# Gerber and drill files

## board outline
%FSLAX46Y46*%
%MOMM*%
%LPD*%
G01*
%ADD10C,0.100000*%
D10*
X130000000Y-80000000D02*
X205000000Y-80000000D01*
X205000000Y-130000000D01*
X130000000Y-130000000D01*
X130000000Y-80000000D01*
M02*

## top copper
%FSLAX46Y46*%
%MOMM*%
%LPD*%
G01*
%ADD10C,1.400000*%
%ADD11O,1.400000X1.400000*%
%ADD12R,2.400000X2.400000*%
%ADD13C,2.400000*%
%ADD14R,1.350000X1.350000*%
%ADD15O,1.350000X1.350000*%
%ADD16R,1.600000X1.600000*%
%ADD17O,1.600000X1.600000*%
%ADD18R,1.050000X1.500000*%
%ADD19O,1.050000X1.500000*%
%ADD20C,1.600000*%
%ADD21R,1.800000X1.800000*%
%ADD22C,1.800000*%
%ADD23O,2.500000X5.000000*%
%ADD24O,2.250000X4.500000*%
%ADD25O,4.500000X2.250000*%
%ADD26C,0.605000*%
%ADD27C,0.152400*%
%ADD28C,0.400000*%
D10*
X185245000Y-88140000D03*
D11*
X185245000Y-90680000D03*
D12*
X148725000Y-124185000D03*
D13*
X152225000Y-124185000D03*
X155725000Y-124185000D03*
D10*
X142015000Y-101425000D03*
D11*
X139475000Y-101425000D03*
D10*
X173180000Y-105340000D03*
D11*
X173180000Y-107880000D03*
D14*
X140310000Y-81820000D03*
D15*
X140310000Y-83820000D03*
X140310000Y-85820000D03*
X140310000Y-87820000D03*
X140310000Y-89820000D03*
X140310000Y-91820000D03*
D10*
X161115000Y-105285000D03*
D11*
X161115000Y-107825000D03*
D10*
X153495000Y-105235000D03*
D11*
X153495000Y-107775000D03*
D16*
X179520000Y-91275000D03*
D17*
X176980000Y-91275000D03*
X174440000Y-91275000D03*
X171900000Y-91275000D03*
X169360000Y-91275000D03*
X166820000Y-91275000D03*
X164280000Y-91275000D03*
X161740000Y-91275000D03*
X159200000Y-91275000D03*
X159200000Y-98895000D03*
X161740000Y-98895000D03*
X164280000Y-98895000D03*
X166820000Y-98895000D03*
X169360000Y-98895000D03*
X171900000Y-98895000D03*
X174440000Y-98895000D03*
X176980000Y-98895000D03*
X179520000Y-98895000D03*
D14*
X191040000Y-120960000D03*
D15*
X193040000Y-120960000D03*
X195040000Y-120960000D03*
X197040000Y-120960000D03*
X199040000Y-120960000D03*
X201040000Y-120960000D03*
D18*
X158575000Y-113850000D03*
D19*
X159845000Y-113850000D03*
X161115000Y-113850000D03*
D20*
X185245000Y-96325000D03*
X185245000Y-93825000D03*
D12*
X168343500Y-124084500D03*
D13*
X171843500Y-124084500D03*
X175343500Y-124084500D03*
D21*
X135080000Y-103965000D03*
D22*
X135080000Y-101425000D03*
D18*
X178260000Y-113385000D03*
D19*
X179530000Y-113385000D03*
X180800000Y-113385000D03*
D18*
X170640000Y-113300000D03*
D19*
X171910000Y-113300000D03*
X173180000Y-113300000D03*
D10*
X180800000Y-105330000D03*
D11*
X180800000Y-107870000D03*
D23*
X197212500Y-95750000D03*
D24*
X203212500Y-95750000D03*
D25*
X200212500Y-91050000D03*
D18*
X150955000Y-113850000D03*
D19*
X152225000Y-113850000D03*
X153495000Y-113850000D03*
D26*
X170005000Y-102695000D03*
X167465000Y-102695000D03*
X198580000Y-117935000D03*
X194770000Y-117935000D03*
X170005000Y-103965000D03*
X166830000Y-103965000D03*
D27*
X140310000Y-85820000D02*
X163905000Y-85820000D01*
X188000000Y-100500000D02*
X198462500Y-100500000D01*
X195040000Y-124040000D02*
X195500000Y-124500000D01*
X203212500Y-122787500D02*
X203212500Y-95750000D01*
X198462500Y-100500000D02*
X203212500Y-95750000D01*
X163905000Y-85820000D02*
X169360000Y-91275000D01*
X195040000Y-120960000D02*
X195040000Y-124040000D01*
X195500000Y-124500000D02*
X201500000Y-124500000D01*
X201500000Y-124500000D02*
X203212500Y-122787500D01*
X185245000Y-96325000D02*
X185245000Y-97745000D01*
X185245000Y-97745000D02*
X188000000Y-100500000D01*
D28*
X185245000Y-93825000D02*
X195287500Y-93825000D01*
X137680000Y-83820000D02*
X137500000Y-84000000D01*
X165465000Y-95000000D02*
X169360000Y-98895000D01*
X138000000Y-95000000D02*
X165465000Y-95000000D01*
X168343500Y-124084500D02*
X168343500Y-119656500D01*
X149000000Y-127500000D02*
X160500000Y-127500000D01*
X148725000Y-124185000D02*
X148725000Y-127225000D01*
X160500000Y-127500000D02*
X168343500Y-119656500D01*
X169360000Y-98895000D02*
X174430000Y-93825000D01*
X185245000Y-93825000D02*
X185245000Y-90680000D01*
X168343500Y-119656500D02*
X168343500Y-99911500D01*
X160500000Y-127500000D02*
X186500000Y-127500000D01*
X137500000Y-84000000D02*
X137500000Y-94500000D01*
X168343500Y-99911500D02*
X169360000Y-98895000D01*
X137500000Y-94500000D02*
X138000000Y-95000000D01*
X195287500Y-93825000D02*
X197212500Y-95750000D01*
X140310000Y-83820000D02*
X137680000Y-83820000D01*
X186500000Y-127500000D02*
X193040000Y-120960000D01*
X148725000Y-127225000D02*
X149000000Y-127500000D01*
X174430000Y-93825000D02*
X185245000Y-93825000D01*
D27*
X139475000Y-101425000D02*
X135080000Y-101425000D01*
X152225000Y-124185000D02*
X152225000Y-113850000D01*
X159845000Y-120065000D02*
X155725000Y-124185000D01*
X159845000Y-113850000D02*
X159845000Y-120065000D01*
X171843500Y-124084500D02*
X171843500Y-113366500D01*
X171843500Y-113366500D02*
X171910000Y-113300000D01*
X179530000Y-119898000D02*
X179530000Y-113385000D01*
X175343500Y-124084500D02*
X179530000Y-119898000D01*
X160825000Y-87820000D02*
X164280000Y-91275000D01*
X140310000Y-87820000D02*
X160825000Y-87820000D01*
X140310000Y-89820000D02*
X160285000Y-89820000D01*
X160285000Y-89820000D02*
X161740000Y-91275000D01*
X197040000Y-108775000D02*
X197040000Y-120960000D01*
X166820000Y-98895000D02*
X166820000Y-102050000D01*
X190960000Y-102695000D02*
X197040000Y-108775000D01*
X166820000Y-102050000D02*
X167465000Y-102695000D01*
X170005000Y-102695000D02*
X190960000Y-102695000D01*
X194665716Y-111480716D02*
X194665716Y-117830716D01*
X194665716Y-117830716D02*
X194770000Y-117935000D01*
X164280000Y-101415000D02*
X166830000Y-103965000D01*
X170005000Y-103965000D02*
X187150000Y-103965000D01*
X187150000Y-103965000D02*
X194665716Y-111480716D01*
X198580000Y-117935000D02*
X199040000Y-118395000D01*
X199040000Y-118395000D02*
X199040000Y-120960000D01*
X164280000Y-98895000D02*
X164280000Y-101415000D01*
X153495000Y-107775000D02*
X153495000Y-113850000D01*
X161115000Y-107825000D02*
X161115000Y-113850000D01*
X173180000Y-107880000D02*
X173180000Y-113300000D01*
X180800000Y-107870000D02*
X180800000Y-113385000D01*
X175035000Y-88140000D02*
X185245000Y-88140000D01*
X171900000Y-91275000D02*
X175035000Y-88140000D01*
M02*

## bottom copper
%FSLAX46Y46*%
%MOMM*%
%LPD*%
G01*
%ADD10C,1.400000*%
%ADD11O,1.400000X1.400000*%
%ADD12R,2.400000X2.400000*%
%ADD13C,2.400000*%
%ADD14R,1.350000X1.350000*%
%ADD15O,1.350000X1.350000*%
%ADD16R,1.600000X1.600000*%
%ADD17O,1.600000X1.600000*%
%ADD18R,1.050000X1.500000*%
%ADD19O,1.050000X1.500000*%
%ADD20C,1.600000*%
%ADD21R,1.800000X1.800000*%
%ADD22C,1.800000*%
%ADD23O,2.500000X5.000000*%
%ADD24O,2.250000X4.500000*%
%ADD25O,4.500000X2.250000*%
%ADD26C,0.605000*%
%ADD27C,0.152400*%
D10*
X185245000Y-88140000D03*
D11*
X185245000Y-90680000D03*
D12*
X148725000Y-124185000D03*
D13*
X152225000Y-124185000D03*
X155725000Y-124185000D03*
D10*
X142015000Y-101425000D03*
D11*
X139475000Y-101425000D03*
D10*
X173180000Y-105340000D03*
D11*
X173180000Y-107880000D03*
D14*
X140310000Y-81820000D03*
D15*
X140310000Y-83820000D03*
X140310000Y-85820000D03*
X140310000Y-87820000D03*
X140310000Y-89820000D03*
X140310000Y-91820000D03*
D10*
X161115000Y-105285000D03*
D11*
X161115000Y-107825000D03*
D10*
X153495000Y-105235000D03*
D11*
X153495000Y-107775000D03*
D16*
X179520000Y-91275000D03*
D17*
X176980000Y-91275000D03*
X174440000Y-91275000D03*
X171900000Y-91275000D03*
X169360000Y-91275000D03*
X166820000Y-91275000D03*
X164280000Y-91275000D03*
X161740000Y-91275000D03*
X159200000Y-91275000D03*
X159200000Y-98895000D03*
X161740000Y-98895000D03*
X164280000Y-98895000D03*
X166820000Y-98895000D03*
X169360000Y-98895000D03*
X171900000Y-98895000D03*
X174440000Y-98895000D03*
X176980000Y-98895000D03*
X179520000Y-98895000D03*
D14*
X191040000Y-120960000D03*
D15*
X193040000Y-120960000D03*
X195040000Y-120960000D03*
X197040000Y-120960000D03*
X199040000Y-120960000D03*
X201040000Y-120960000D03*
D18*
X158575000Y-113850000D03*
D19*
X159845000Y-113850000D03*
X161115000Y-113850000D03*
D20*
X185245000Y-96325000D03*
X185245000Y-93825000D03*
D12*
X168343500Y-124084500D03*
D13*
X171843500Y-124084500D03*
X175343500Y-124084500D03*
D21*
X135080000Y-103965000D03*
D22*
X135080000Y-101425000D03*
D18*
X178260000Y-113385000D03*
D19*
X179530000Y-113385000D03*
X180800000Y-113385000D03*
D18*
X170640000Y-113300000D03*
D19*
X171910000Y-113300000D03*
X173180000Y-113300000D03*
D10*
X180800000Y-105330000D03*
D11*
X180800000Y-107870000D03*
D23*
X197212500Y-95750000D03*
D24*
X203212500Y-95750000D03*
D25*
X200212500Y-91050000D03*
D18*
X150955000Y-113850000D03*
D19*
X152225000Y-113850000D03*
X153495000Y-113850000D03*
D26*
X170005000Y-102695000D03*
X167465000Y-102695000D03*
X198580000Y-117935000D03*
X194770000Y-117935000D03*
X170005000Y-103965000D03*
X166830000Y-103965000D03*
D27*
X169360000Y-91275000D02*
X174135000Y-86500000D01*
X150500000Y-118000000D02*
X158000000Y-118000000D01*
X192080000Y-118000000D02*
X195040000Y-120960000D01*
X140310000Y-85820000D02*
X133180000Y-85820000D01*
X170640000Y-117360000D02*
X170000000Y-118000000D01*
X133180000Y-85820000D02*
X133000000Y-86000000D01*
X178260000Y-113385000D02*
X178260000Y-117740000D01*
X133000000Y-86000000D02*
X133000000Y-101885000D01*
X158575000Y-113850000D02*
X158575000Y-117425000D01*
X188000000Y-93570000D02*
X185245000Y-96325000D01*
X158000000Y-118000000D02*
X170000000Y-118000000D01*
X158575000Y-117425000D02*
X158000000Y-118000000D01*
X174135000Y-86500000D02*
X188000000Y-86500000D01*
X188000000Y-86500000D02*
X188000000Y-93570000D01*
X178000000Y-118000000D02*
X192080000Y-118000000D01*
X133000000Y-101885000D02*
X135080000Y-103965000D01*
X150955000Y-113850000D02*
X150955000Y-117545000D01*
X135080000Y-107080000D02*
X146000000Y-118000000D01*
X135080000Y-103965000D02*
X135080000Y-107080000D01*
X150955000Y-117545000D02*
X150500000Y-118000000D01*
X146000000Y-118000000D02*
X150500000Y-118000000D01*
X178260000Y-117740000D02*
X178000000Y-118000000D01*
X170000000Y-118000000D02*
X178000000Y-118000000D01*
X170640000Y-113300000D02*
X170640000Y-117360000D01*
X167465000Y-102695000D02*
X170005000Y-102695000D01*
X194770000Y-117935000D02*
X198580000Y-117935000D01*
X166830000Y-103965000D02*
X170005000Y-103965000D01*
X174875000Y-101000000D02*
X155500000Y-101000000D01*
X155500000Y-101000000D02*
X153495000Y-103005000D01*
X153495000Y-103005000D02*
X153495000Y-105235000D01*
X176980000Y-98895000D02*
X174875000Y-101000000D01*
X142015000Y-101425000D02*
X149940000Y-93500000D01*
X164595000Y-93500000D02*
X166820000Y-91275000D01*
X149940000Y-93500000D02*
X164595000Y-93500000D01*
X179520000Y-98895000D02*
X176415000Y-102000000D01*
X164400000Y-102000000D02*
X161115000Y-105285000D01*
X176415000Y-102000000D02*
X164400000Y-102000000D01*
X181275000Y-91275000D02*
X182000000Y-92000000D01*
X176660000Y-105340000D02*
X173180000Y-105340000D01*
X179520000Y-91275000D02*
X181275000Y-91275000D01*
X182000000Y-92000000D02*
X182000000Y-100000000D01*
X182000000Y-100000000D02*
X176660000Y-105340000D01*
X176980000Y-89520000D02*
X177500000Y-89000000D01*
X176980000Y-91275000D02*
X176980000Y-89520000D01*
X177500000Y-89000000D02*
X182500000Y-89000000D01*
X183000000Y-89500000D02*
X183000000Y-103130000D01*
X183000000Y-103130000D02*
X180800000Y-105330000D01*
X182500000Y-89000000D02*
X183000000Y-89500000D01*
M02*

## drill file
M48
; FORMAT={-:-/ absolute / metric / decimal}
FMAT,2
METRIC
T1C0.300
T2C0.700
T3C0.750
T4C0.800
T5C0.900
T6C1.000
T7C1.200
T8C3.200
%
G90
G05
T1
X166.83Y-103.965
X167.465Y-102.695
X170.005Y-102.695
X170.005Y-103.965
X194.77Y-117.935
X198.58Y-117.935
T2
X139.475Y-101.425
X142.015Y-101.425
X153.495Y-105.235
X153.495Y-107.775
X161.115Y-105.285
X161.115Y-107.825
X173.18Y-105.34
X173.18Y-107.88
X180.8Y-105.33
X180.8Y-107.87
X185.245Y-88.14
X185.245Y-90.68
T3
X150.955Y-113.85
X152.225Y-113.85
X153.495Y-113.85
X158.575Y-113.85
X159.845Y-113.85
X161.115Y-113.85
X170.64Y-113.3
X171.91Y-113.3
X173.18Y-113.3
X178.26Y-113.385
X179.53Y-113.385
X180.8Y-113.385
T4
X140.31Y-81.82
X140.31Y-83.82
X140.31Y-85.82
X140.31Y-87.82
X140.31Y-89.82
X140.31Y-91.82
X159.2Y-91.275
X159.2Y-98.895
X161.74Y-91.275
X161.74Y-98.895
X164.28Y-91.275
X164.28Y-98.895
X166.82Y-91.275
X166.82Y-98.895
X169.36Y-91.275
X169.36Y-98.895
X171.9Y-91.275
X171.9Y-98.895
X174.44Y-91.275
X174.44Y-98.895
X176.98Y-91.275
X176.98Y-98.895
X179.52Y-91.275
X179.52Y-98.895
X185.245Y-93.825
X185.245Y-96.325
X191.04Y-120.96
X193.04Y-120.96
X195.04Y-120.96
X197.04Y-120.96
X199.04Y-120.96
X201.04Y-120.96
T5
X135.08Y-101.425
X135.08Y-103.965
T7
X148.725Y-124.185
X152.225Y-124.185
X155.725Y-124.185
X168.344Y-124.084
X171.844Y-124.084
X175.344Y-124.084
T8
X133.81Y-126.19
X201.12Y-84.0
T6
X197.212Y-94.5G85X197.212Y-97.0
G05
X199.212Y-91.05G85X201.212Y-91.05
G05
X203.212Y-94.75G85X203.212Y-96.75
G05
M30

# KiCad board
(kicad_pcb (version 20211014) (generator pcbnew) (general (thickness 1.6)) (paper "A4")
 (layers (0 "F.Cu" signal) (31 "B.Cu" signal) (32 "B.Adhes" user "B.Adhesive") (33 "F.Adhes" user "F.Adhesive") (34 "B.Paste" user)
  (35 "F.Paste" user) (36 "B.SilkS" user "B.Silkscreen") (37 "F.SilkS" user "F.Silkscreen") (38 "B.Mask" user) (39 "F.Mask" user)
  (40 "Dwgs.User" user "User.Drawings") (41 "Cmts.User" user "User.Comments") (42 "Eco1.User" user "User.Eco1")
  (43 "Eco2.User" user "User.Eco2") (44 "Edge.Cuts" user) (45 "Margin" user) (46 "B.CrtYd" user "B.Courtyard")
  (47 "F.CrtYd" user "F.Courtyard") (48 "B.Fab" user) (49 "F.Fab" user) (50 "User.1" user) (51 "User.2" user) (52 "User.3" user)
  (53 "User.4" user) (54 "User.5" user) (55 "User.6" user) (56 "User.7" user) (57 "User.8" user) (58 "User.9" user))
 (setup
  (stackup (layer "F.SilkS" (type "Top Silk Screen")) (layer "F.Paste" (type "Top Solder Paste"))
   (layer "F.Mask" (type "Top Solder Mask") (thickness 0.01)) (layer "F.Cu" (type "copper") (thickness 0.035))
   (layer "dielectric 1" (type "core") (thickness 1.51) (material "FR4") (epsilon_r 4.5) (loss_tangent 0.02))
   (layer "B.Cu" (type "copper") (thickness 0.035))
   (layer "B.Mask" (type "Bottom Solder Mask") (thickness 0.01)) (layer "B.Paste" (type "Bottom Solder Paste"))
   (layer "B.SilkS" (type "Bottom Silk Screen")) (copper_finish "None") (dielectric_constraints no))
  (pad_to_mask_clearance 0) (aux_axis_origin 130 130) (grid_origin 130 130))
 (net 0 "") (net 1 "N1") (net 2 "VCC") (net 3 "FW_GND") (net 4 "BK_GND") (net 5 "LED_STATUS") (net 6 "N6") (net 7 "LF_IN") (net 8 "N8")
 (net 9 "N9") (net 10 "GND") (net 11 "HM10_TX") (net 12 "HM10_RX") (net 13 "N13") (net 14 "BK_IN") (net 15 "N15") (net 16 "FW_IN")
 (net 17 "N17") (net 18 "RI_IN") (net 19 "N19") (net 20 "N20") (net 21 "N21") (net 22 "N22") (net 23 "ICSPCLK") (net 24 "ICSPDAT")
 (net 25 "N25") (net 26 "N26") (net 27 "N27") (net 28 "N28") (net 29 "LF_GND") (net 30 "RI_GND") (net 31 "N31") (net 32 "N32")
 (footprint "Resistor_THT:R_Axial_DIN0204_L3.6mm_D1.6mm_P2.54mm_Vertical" (layer "F.Cu") (at 185.245 88.14 -90)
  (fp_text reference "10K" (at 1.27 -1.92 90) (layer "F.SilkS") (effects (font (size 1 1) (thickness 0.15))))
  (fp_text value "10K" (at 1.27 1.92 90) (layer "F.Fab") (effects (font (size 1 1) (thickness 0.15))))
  (pad "1" thru_hole circle (at 0 0 270) (size 1.4 1.4) (drill 0.7) (layers *.Cu *.Mask) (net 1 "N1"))
  (pad "2" thru_hole oval (at 2.54 0 270) (size 1.4 1.4) (drill 0.7) (layers *.Cu *.Mask) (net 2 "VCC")))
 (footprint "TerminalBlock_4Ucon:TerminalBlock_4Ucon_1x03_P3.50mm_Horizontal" (layer "F.Cu") (at 148.725 124.185)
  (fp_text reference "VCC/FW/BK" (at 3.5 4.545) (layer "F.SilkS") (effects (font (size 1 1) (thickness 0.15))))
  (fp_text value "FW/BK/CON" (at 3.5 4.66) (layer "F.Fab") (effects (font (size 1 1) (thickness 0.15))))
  (pad "1" thru_hole rect (at 0 0) (size 2.4 2.4) (drill 1.2) (layers *.Cu *.Mask) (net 2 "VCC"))
  (pad "2" thru_hole circle (at 3.5 0) (size 2.4 2.4) (drill 1.2) (layers *.Cu *.Mask) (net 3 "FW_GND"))
  (pad "3" thru_hole circle (at 7 0) (size 2.4 2.4) (drill 1.2) (layers *.Cu *.Mask) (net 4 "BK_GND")))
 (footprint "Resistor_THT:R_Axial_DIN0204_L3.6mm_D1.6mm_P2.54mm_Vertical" (layer "F.Cu") (at 142.015 101.425 180)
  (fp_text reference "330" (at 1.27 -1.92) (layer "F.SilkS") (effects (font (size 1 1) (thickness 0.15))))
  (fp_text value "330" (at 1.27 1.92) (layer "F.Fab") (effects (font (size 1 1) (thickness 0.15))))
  (pad "1" thru_hole circle (at 0 0 180) (size 1.4 1.4) (drill 0.7) (layers *.Cu *.Mask) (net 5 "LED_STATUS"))
  (pad "2" thru_hole oval (at 2.54 0 180) (size 1.4 1.4) (drill 0.7) (layers *.Cu *.Mask) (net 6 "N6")))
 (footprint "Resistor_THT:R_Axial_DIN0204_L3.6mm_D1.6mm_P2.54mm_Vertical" (layer "F.Cu") (at 173.18 105.34 -90)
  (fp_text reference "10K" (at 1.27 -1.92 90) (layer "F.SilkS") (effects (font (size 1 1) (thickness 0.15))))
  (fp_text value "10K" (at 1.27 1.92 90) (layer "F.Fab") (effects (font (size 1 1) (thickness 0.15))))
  (pad "1" thru_hole circle (at 0 0 270) (size 1.4 1.4) (drill 0.7) (layers *.Cu *.Mask) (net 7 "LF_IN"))
  (pad "2" thru_hole oval (at 2.54 0 270) (size 1.4 1.4) (drill 0.7) (layers *.Cu *.Mask) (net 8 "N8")))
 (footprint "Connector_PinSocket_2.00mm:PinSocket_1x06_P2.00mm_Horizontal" (layer "F.Cu") (at 140.31 81.82)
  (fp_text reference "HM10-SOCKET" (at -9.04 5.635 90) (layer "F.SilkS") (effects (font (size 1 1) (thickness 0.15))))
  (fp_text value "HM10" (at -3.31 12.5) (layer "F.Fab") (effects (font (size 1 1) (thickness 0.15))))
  (pad "1" thru_hole rect (at 0 0) (size 1.35 1.35) (drill 0.8) (layers *.Cu *.Mask) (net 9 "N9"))
  (pad "2" thru_hole oval (at 0 2) (size 1.35 1.35) (drill 0.8) (layers *.Cu *.Mask) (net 2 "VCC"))
  (pad "3" thru_hole oval (at 0 4) (size 1.35 1.35) (drill 0.8) (layers *.Cu *.Mask) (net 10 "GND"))
  (pad "4" thru_hole oval (at 0 6) (size 1.35 1.35) (drill 0.8) (layers *.Cu *.Mask) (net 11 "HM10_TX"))
  (pad "5" thru_hole oval (at 0 8) (size 1.35 1.35) (drill 0.8) (layers *.Cu *.Mask) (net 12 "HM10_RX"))
  (pad "6" thru_hole oval (at 0 10) (size 1.35 1.35) (drill 0.8) (layers *.Cu *.Mask) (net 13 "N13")))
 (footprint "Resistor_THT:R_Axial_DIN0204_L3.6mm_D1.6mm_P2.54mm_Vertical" (layer "F.Cu") (at 161.115 105.285 -90)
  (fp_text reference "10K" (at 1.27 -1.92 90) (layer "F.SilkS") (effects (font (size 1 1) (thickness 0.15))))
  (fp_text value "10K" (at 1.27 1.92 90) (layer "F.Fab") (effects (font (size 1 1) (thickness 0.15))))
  (pad "1" thru_hole circle (at 0 0 270) (size 1.4 1.4) (drill 0.7) (layers *.Cu *.Mask) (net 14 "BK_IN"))
  (pad "2" thru_hole oval (at 2.54 0 270) (size 1.4 1.4) (drill 0.7) (layers *.Cu *.Mask) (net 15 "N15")))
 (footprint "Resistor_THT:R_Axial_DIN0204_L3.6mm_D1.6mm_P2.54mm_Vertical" (layer "F.Cu") (at 153.495 105.235 -90)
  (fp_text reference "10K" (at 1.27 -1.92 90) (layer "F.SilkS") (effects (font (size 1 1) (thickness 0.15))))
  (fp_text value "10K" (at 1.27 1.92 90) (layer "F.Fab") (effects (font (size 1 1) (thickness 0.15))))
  (pad "1" thru_hole circle (at 0 0 270) (size 1.4 1.4) (drill 0.7) (layers *.Cu *.Mask) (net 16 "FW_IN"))
  (pad "2" thru_hole oval (at 2.54 0 270) (size 1.4 1.4) (drill 0.7) (layers *.Cu *.Mask) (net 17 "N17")))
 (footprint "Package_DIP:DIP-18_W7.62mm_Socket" (layer "F.Cu") (at 179.52 91.275 -90)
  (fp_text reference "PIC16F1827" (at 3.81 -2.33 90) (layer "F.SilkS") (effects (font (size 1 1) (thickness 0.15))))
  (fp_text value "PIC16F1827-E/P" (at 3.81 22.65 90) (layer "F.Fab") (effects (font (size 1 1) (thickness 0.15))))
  (pad "1" thru_hole rect (at 0 0 270) (size 1.6 1.6) (drill 0.8) (layers *.Cu *.Mask) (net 7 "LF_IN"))
  (pad "2" thru_hole oval (at 0 2.54 270) (size 1.6 1.6) (drill 0.8) (layers *.Cu *.Mask) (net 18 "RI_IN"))
  (pad "3" thru_hole oval (at 0 5.08 270) (size 1.6 1.6) (drill 0.8) (layers *.Cu *.Mask) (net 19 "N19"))
  (pad "4" thru_hole oval (at 0 7.62 270) (size 1.6 1.6) (drill 0.8) (layers *.Cu *.Mask) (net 1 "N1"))
  (pad "5" thru_hole oval (at 0 10.16 270) (size 1.6 1.6) (drill 0.8) (layers *.Cu *.Mask) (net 10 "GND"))
  (pad "6" thru_hole oval (at 0 12.7 270) (size 1.6 1.6) (drill 0.8) (layers *.Cu *.Mask) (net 5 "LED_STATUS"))
  (pad "7" thru_hole oval (at 0 15.24 270) (size 1.6 1.6) (drill 0.8) (layers *.Cu *.Mask) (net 11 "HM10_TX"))
  (pad "8" thru_hole oval (at 0 17.78 270) (size 1.6 1.6) (drill 0.8) (layers *.Cu *.Mask) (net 12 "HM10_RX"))
  (pad "9" thru_hole oval (at 0 20.32 270) (size 1.6 1.6) (drill 0.8) (layers *.Cu *.Mask) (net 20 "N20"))
  (pad "10" thru_hole oval (at 7.62 20.32 270) (size 1.6 1.6) (drill 0.8) (layers *.Cu *.Mask) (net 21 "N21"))
  (pad "11" thru_hole oval (at 7.62 17.78 270) (size 1.6 1.6) (drill 0.8) (layers *.Cu *.Mask) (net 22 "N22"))
  (pad "12" thru_hole oval (at 7.62 15.24 270) (size 1.6 1.6) (drill 0.8) (layers *.Cu *.Mask) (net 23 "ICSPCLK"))
  (pad "13" thru_hole oval (at 7.62 12.7 270) (size 1.6 1.6) (drill 0.8) (layers *.Cu *.Mask) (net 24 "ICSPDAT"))
  (pad "14" thru_hole oval (at 7.62 10.16 270) (size 1.6 1.6) (drill 0.8) (layers *.Cu *.Mask) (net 2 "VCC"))
  (pad "15" thru_hole oval (at 7.62 7.62 270) (size 1.6 1.6) (drill 0.8) (layers *.Cu *.Mask) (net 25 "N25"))
  (pad "16" thru_hole oval (at 7.62 5.08 270) (size 1.6 1.6) (drill 0.8) (layers *.Cu *.Mask) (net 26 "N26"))
  (pad "17" thru_hole oval (at 7.62 2.54 270) (size 1.6 1.6) (drill 0.8) (layers *.Cu *.Mask) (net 16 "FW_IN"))
  (pad "18" thru_hole oval (at 7.62 0 270) (size 1.6 1.6) (drill 0.8) (layers *.Cu *.Mask) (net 14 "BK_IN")))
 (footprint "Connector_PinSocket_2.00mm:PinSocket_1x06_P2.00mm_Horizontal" (layer "F.Cu") (at 191.04 120.96 90)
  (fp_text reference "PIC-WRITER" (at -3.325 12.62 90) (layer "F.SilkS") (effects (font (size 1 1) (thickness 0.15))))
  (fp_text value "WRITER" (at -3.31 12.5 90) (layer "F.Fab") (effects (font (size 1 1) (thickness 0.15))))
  (pad "1" thru_hole rect (at 0 0 90) (size 1.35 1.35) (drill 0.8) (layers *.Cu *.Mask) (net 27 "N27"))
  (pad "2" thru_hole oval (at 0 2 90) (size 1.35 1.35) (drill 0.8) (layers *.Cu *.Mask) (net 2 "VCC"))
  (pad "3" thru_hole oval (at 0 4 90) (size 1.35 1.35) (drill 0.8) (layers *.Cu *.Mask) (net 10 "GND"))
  (pad "4" thru_hole oval (at 0 6 90) (size 1.35 1.35) (drill 0.8) (layers *.Cu *.Mask) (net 24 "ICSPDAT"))
  (pad "5" thru_hole oval (at 0 8 90) (size 1.35 1.35) (drill 0.8) (layers *.Cu *.Mask) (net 23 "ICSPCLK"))
  (pad "6" thru_hole oval (at 0 10 90) (size 1.35 1.35) (drill 0.8) (layers *.Cu *.Mask) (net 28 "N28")))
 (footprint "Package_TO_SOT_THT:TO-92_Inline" (layer "F.Cu") (at 158.575 113.85)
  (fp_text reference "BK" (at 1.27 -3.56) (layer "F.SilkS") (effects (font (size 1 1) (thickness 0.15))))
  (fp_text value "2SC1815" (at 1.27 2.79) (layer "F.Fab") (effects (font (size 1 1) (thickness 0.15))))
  (pad "1" thru_hole rect (at 0 0) (size 1.05 1.5) (drill 0.75) (layers *.Cu *.Mask) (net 10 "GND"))
  (pad "2" thru_hole oval (at 1.27 0) (size 1.05 1.5) (drill 0.75) (layers *.Cu *.Mask) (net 4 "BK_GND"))
  (pad "3" thru_hole oval (at 2.54 0) (size 1.05 1.5) (drill 0.75) (layers *.Cu *.Mask) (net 15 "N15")))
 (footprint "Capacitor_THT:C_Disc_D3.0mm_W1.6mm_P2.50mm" (layer "F.Cu") (at 185.245 96.325 90)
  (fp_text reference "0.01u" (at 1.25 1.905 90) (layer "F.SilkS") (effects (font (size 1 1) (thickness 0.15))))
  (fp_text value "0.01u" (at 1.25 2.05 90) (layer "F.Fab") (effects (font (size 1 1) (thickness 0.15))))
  (pad "1" thru_hole circle (at 0 0 90) (size 1.6 1.6) (drill 0.8) (layers *.Cu *.Mask) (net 10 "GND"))
  (pad "2" thru_hole circle (at 2.5 0 90) (size 1.6 1.6) (drill 0.8) (layers *.Cu *.Mask) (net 2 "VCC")))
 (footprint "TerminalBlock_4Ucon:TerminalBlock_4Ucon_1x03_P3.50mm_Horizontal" (layer "F.Cu") (at 168.3435 124.0845)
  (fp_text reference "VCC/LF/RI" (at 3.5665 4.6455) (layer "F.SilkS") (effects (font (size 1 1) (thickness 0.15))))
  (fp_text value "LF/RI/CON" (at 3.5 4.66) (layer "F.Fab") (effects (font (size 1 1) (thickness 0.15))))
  (pad "1" thru_hole rect (at 0 0) (size 2.4 2.4) (drill 1.2) (layers *.Cu *.Mask) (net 2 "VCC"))
  (pad "2" thru_hole circle (at 3.5 0) (size 2.4 2.4) (drill 1.2) (layers *.Cu *.Mask) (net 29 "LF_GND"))
  (pad "3" thru_hole circle (at 7 0) (size 2.4 2.4) (drill 1.2) (layers *.Cu *.Mask) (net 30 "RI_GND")))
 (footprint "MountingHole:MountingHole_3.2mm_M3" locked (layer "F.Cu") (at 201.12 84)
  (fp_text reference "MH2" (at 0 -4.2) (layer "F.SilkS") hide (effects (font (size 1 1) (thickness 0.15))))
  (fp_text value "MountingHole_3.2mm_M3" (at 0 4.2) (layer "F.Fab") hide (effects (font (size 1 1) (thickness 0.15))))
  (pad "" np_thru_hole circle locked (at 0 0) (size 3.2 3.2) (drill 3.2) (layers *.Cu *.Mask)))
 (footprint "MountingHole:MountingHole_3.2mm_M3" (layer "F.Cu") (at 133.81 126.19)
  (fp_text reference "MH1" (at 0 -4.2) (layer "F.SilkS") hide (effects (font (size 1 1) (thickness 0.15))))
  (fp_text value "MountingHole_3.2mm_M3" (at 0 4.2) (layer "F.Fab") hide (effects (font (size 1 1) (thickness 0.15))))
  (pad "" np_thru_hole circle (at 0 0) (size 3.2 3.2) (drill 3.2) (layers F&B.Cu *.Mask)))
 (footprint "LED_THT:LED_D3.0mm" (layer "F.Cu") (at 135.08 103.965 90)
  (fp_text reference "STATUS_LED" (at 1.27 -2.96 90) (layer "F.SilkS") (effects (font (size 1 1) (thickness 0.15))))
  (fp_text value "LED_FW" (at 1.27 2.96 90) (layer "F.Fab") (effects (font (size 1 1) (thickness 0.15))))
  (pad "1" thru_hole rect (at 0 0 90) (size 1.8 1.8) (drill 0.9) (layers *.Cu *.Mask) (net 10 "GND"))
  (pad "2" thru_hole circle (at 2.54 0 90) (size 1.8 1.8) (drill 0.9) (layers *.Cu *.Mask) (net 6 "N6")))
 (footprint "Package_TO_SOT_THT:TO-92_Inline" (layer "F.Cu") (at 178.26 113.385)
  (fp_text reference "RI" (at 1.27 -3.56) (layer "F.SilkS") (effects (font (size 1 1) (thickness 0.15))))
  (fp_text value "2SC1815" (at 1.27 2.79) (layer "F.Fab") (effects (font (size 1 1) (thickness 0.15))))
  (pad "1" thru_hole rect (at 0 0) (size 1.05 1.5) (drill 0.75) (layers *.Cu *.Mask) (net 10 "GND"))
  (pad "2" thru_hole oval (at 1.27 0) (size 1.05 1.5) (drill 0.75) (layers *.Cu *.Mask) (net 30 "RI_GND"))
  (pad "3" thru_hole oval (at 2.54 0) (size 1.05 1.5) (drill 0.75) (layers *.Cu *.Mask) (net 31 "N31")))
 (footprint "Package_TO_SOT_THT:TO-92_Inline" (layer "F.Cu") (at 170.64 113.3)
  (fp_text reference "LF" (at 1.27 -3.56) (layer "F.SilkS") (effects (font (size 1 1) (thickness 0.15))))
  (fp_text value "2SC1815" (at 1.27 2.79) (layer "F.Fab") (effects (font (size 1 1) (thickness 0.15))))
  (pad "1" thru_hole rect (at 0 0) (size 1.05 1.5) (drill 0.75) (layers *.Cu *.Mask) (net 10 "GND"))
  (pad "2" thru_hole oval (at 1.27 0) (size 1.05 1.5) (drill 0.75) (layers *.Cu *.Mask) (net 29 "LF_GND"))
  (pad "3" thru_hole oval (at 2.54 0) (size 1.05 1.5) (drill 0.75) (layers *.Cu *.Mask) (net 8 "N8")))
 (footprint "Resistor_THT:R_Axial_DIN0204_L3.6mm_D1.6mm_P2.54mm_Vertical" (layer "F.Cu") (at 180.8 105.33 -90)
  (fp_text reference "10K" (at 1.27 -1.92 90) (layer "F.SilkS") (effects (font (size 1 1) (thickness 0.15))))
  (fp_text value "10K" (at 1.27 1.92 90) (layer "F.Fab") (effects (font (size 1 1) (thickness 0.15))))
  (pad "1" thru_hole circle (at 0 0 270) (size 1.4 1.4) (drill 0.7) (layers *.Cu *.Mask) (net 18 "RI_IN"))
  (pad "2" thru_hole oval (at 2.54 0 270) (size 1.4 1.4) (drill 0.7) (layers *.Cu *.Mask) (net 31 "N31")))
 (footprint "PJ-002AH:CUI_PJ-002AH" (layer "F.Cu") (at 197.2125 95.75)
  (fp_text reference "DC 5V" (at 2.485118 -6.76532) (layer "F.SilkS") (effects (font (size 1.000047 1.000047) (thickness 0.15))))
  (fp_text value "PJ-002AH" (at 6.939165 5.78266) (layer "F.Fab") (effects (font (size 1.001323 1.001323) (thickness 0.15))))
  (pad "1" thru_hole oval locked (at 0 0) (size 2.5 5) (drill oval 1 3.5) (layers *.Cu *.Mask) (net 2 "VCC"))
  (pad "2" thru_hole oval locked (at 6 0) (size 2.25 4.5) (drill oval 1 3) (layers *.Cu *.Mask) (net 10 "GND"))
  (pad "3" thru_hole oval locked (at 3 -4.7) (size 4.5 2.25) (drill oval 3 1) (layers *.Cu *.Mask) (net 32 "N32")))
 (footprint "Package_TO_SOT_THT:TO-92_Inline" (layer "F.Cu") (at 150.955 113.85)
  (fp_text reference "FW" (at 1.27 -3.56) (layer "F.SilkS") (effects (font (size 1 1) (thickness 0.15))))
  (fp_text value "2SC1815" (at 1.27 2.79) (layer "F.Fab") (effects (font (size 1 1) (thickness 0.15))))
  (pad "1" thru_hole rect (at 0 0) (size 1.05 1.5) (drill 0.75) (layers *.Cu *.Mask) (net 10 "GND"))
  (pad "2" thru_hole oval (at 1.27 0) (size 1.05 1.5) (drill 0.75) (layers *.Cu *.Mask) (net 3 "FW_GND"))
  (pad "3" thru_hole oval (at 2.54 0) (size 1.05 1.5) (drill 0.75) (layers *.Cu *.Mask) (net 17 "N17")))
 (gr_rect locked (start 130 130) (end 205 80) (layer "Edge.Cuts") (width 0.1) (fill none))
 (segment (start 140.31 85.82) (end 163.905 85.82) (width 0.1524) (layer "F.Cu") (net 10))
 (segment (start 188 100.5) (end 198.4625 100.5) (width 0.1524) (layer "F.Cu") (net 10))
 (segment (start 195.04 124.04) (end 195.5 124.5) (width 0.1524) (layer "F.Cu") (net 10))
 (segment (start 203.2125 122.7875) (end 203.2125 95.75) (width 0.1524) (layer "F.Cu") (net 10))
 (segment (start 198.4625 100.5) (end 203.2125 95.75) (width 0.1524) (layer "F.Cu") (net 10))
 (segment (start 163.905 85.82) (end 169.36 91.275) (width 0.1524) (layer "F.Cu") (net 10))
 (segment (start 195.04 120.96) (end 195.04 124.04) (width 0.1524) (layer "F.Cu") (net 10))
 (segment (start 195.5 124.5) (end 201.5 124.5) (width 0.1524) (layer "F.Cu") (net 10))
 (segment (start 201.5 124.5) (end 203.2125 122.7875) (width 0.1524) (layer "F.Cu") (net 10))
 (segment (start 185.245 96.325) (end 185.245 97.745) (width 0.1524) (layer "F.Cu") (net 10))
 (segment (start 185.245 97.745) (end 188 100.5) (width 0.1524) (layer "F.Cu") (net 10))
 (segment (start 169.36 91.275) (end 174.135 86.5) (width 0.1524) (layer "B.Cu") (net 10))
 (segment (start 150.5 118) (end 158 118) (width 0.1524) (layer "B.Cu") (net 10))
 (segment (start 192.08 118) (end 195.04 120.96) (width 0.1524) (layer "B.Cu") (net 10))
 (segment (start 140.31 85.82) (end 133.18 85.82) (width 0.1524) (layer "B.Cu") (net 10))
 (segment (start 170.64 117.36) (end 170 118) (width 0.1524) (layer "B.Cu") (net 10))
 (segment (start 133.18 85.82) (end 133 86) (width 0.1524) (layer "B.Cu") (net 10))
 (segment (start 178.26 113.385) (end 178.26 117.74) (width 0.1524) (layer "B.Cu") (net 10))
 (segment (start 133 86) (end 133 101.885) (width 0.1524) (layer "B.Cu") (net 10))
 (segment (start 158.575 113.85) (end 158.575 117.425) (width 0.1524) (layer "B.Cu") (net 10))
 (segment (start 188 93.57) (end 185.245 96.325) (width 0.1524) (layer "B.Cu") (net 10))
 (segment (start 158 118) (end 170 118) (width 0.1524) (layer "B.Cu") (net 10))
 (segment (start 158.575 117.425) (end 158 118) (width 0.1524) (layer "B.Cu") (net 10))
 (segment (start 174.135 86.5) (end 188 86.5) (width 0.1524) (layer "B.Cu") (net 10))
 (segment (start 188 86.5) (end 188 93.57) (width 0.1524) (layer "B.Cu") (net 10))
 (segment (start 178 118) (end 192.08 118) (width 0.1524) (layer "B.Cu") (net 10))
 (segment (start 133 101.885) (end 135.08 103.965) (width 0.1524) (layer "B.Cu") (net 10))
 (segment (start 150.955 113.85) (end 150.955 117.545) (width 0.1524) (layer "B.Cu") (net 10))
 (segment (start 135.08 107.08) (end 146 118) (width 0.1524) (layer "B.Cu") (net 10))
 (segment (start 135.08 103.965) (end 135.08 107.08) (width 0.1524) (layer "B.Cu") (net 10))
 (segment (start 150.955 117.545) (end 150.5 118) (width 0.1524) (layer "B.Cu") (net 10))
 (segment (start 146 118) (end 150.5 118) (width 0.1524) (layer "B.Cu") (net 10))
 (segment (start 178.26 117.74) (end 178 118) (width 0.1524) (layer "B.Cu") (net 10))
 (segment (start 170 118) (end 178 118) (width 0.1524) (layer "B.Cu") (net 10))
 (segment (start 170.64 113.3) (end 170.64 117.36) (width 0.1524) (layer "B.Cu") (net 10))
 (segment (start 185.245 93.825) (end 195.2875 93.825) (width 0.4) (layer "F.Cu") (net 2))
 (segment (start 137.68 83.82) (end 137.5 84) (width 0.4) (layer "F.Cu") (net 2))
 (segment (start 165.465 95) (end 169.36 98.895) (width 0.4) (layer "F.Cu") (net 2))
 (segment (start 138 95) (end 165.465 95) (width 0.4) (layer "F.Cu") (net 2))
 (segment (start 168.3435 124.0845) (end 168.3435 119.6565) (width 0.4) (layer "F.Cu") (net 2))
 (segment (start 149 127.5) (end 160.5 127.5) (width 0.4) (layer "F.Cu") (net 2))
 (segment (start 148.725 124.185) (end 148.725 127.225) (width 0.4) (layer "F.Cu") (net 2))
 (segment (start 160.5 127.5) (end 168.3435 119.6565) (width 0.4) (layer "F.Cu") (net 2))
 (segment (start 169.36 98.895) (end 174.43 93.825) (width 0.4) (layer "F.Cu") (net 2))
 (segment (start 185.245 93.825) (end 185.245 90.68) (width 0.4) (layer "F.Cu") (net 2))
 (segment (start 168.3435 119.6565) (end 168.3435 99.9115) (width 0.4) (layer "F.Cu") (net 2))
 (segment (start 160.5 127.5) (end 186.5 127.5) (width 0.4) (layer "F.Cu") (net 2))
 (segment (start 137.5 84) (end 137.5 94.5) (width 0.4) (layer "F.Cu") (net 2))
 (segment (start 168.3435 99.9115) (end 169.36 98.895) (width 0.4) (layer "F.Cu") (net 2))
 (segment (start 137.5 94.5) (end 138 95) (width 0.4) (layer "F.Cu") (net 2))
 (segment (start 195.2875 93.825) (end 197.2125 95.75) (width 0.4) (layer "F.Cu") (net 2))
 (segment (start 140.31 83.82) (end 137.68 83.82) (width 0.4) (layer "F.Cu") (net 2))
 (segment (start 186.5 127.5) (end 193.04 120.96) (width 0.4) (layer "F.Cu") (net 2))
 (segment (start 148.725 127.225) (end 149 127.5) (width 0.4) (layer "F.Cu") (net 2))
 (segment (start 174.43 93.825) (end 185.245 93.825) (width 0.4) (layer "F.Cu") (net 2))
 (segment (start 139.475 101.425) (end 135.08 101.425) (width 0.1524) (layer "F.Cu") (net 6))
 (segment (start 152.225 124.185) (end 152.225 113.85) (width 0.1524) (layer "F.Cu") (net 3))
 (segment (start 159.845 120.065) (end 155.725 124.185) (width 0.1524) (layer "F.Cu") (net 4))
 (segment (start 159.845 113.85) (end 159.845 120.065) (width 0.1524) (layer "F.Cu") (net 4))
 (segment (start 171.8435 124.0845) (end 171.8435 113.3665) (width 0.1524) (layer "F.Cu") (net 29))
 (segment (start 171.8435 113.3665) (end 171.91 113.3) (width 0.1524) (layer "F.Cu") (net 29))
 (segment (start 179.53 119.898) (end 179.53 113.385) (width 0.1524) (layer "F.Cu") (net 30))
 (segment (start 175.3435 124.0845) (end 179.53 119.898) (width 0.1524) (layer "F.Cu") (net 30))
 (segment (start 160.825 87.82) (end 164.28 91.275) (width 0.1524) (layer "F.Cu") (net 11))
 (segment (start 140.31 87.82) (end 160.825 87.82) (width 0.1524) (layer "F.Cu") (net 11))
 (segment (start 140.31 89.82) (end 160.285 89.82) (width 0.1524) (layer "F.Cu") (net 12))
 (segment (start 160.285 89.82) (end 161.74 91.275) (width 0.1524) (layer "F.Cu") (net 12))
 (segment (start 197.04 108.775) (end 197.04 120.96) (width 0.1524) (layer "F.Cu") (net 24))
 (segment (start 166.82 98.895) (end 166.82 102.05) (width 0.1524) (layer "F.Cu") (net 24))
 (segment (start 190.96 102.695) (end 197.04 108.775) (width 0.1524) (layer "F.Cu") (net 24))
 (segment (start 166.82 102.05) (end 167.465 102.695) (width 0.1524) (layer "F.Cu") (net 24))
 (segment (start 170.005 102.695) (end 190.96 102.695) (width 0.1524) (layer "F.Cu") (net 24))
 (via (at 170.005 102.695) (size 0.605) (drill 0.3) (layers "F.Cu" "B.Cu") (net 24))
 (via (at 167.465 102.695) (size 0.605) (drill 0.3) (layers "F.Cu" "B.Cu") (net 24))
 (segment (start 167.465 102.695) (end 170.005 102.695) (width 0.1524) (layer "B.Cu") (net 24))
 (segment (start 194.665716 111.480716) (end 194.665716 117.830716) (width 0.1524) (layer "F.Cu") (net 23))
 (segment (start 194.665716 117.830716) (end 194.77 117.935) (width 0.1524) (layer "F.Cu") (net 23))
 (segment (start 164.28 101.415) (end 166.83 103.965) (width 0.1524) (layer "F.Cu") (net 23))
 (segment (start 170.005 103.965) (end 187.15 103.965) (width 0.1524) (layer "F.Cu") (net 23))
 (segment (start 187.15 103.965) (end 194.665716 111.480716) (width 0.1524) (layer "F.Cu") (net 23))
 (segment (start 198.58 117.935) (end 199.04 118.395) (width 0.1524) (layer "F.Cu") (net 23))
 (segment (start 199.04 118.395) (end 199.04 120.96) (width 0.1524) (layer "F.Cu") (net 23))
 (segment (start 164.28 98.895) (end 164.28 101.415) (width 0.1524) (layer "F.Cu") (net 23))
 (via (at 198.58 117.935) (size 0.605) (drill 0.3) (layers "F.Cu" "B.Cu") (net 23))
 (via (at 194.77 117.935) (size 0.605) (drill 0.3) (layers "F.Cu" "B.Cu") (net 23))
 (via (at 170.005 103.965) (size 0.605) (drill 0.3) (layers "F.Cu" "B.Cu") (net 23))
 (via (at 166.83 103.965) (size 0.605) (drill 0.3) (layers "F.Cu" "B.Cu") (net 23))
 (segment (start 194.77 117.935) (end 198.58 117.935) (width 0.1524) (layer "B.Cu") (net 23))
 (segment (start 166.83 103.965) (end 170.005 103.965) (width 0.1524) (layer "B.Cu") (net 23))
 (segment (start 153.495 107.775) (end 153.495 113.85) (width 0.1524) (layer "F.Cu") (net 17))
 (segment (start 161.115 107.825) (end 161.115 113.85) (width 0.1524) (layer "F.Cu") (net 15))
 (segment (start 173.18 107.88) (end 173.18 113.3) (width 0.1524) (layer "F.Cu") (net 8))
 (segment (start 180.8 107.87) (end 180.8 113.385) (width 0.1524) (layer "F.Cu") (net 31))
 (segment (start 175.035 88.14) (end 185.245 88.14) (width 0.1524) (layer "F.Cu") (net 1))
 (segment (start 171.9 91.275) (end 175.035 88.14) (width 0.1524) (layer "F.Cu") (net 1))
 (segment (start 174.875 101) (end 155.5 101) (width 0.1524) (layer "B.Cu") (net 16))
 (segment (start 155.5 101) (end 153.495 103.005) (width 0.1524) (layer "B.Cu") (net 16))
 (segment (start 153.495 103.005) (end 153.495 105.235) (width 0.1524) (layer "B.Cu") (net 16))
 (segment (start 176.98 98.895) (end 174.875 101) (width 0.1524) (layer "B.Cu") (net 16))
 (segment (start 142.015 101.425) (end 149.94 93.5) (width 0.1524) (layer "B.Cu") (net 5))
 (segment (start 164.595 93.5) (end 166.82 91.275) (width 0.1524) (layer "B.Cu") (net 5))
 (segment (start 149.94 93.5) (end 164.595 93.5) (width 0.1524) (layer "B.Cu") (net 5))
 (segment (start 179.52 98.895) (end 176.415 102) (width 0.1524) (layer "B.Cu") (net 14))
 (segment (start 164.4 102) (end 161.115 105.285) (width 0.1524) (layer "B.Cu") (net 14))
 (segment (start 176.415 102) (end 164.4 102) (width 0.1524) (layer "B.Cu") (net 14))
 (segment (start 181.275 91.275) (end 182 92) (width 0.1524) (layer "B.Cu") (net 7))
 (segment (start 176.66 105.34) (end 173.18 105.34) (width 0.1524) (layer "B.Cu") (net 7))
 (segment (start 179.52 91.275) (end 181.275 91.275) (width 0.1524) (layer "B.Cu") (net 7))
 (segment (start 182 92) (end 182 100) (width 0.1524) (layer "B.Cu") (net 7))
 (segment (start 182 100) (end 176.66 105.34) (width 0.1524) (layer "B.Cu") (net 7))
 (segment (start 176.98 89.52) (end 177.5 89) (width 0.1524) (layer "B.Cu") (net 18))
 (segment (start 176.98 91.275) (end 176.98 89.52) (width 0.1524) (layer "B.Cu") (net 18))
 (segment (start 177.5 89) (end 182.5 89) (width 0.1524) (layer "B.Cu") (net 18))
 (segment (start 183 89.5) (end 183 103.13) (width 0.1524) (layer "B.Cu") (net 18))
 (segment (start 183 103.13) (end 180.8 105.33) (width 0.1524) (layer "B.Cu") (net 18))
 (segment (start 182.5 89) (end 183 89.5) (width 0.1524) (layer "B.Cu") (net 18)))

